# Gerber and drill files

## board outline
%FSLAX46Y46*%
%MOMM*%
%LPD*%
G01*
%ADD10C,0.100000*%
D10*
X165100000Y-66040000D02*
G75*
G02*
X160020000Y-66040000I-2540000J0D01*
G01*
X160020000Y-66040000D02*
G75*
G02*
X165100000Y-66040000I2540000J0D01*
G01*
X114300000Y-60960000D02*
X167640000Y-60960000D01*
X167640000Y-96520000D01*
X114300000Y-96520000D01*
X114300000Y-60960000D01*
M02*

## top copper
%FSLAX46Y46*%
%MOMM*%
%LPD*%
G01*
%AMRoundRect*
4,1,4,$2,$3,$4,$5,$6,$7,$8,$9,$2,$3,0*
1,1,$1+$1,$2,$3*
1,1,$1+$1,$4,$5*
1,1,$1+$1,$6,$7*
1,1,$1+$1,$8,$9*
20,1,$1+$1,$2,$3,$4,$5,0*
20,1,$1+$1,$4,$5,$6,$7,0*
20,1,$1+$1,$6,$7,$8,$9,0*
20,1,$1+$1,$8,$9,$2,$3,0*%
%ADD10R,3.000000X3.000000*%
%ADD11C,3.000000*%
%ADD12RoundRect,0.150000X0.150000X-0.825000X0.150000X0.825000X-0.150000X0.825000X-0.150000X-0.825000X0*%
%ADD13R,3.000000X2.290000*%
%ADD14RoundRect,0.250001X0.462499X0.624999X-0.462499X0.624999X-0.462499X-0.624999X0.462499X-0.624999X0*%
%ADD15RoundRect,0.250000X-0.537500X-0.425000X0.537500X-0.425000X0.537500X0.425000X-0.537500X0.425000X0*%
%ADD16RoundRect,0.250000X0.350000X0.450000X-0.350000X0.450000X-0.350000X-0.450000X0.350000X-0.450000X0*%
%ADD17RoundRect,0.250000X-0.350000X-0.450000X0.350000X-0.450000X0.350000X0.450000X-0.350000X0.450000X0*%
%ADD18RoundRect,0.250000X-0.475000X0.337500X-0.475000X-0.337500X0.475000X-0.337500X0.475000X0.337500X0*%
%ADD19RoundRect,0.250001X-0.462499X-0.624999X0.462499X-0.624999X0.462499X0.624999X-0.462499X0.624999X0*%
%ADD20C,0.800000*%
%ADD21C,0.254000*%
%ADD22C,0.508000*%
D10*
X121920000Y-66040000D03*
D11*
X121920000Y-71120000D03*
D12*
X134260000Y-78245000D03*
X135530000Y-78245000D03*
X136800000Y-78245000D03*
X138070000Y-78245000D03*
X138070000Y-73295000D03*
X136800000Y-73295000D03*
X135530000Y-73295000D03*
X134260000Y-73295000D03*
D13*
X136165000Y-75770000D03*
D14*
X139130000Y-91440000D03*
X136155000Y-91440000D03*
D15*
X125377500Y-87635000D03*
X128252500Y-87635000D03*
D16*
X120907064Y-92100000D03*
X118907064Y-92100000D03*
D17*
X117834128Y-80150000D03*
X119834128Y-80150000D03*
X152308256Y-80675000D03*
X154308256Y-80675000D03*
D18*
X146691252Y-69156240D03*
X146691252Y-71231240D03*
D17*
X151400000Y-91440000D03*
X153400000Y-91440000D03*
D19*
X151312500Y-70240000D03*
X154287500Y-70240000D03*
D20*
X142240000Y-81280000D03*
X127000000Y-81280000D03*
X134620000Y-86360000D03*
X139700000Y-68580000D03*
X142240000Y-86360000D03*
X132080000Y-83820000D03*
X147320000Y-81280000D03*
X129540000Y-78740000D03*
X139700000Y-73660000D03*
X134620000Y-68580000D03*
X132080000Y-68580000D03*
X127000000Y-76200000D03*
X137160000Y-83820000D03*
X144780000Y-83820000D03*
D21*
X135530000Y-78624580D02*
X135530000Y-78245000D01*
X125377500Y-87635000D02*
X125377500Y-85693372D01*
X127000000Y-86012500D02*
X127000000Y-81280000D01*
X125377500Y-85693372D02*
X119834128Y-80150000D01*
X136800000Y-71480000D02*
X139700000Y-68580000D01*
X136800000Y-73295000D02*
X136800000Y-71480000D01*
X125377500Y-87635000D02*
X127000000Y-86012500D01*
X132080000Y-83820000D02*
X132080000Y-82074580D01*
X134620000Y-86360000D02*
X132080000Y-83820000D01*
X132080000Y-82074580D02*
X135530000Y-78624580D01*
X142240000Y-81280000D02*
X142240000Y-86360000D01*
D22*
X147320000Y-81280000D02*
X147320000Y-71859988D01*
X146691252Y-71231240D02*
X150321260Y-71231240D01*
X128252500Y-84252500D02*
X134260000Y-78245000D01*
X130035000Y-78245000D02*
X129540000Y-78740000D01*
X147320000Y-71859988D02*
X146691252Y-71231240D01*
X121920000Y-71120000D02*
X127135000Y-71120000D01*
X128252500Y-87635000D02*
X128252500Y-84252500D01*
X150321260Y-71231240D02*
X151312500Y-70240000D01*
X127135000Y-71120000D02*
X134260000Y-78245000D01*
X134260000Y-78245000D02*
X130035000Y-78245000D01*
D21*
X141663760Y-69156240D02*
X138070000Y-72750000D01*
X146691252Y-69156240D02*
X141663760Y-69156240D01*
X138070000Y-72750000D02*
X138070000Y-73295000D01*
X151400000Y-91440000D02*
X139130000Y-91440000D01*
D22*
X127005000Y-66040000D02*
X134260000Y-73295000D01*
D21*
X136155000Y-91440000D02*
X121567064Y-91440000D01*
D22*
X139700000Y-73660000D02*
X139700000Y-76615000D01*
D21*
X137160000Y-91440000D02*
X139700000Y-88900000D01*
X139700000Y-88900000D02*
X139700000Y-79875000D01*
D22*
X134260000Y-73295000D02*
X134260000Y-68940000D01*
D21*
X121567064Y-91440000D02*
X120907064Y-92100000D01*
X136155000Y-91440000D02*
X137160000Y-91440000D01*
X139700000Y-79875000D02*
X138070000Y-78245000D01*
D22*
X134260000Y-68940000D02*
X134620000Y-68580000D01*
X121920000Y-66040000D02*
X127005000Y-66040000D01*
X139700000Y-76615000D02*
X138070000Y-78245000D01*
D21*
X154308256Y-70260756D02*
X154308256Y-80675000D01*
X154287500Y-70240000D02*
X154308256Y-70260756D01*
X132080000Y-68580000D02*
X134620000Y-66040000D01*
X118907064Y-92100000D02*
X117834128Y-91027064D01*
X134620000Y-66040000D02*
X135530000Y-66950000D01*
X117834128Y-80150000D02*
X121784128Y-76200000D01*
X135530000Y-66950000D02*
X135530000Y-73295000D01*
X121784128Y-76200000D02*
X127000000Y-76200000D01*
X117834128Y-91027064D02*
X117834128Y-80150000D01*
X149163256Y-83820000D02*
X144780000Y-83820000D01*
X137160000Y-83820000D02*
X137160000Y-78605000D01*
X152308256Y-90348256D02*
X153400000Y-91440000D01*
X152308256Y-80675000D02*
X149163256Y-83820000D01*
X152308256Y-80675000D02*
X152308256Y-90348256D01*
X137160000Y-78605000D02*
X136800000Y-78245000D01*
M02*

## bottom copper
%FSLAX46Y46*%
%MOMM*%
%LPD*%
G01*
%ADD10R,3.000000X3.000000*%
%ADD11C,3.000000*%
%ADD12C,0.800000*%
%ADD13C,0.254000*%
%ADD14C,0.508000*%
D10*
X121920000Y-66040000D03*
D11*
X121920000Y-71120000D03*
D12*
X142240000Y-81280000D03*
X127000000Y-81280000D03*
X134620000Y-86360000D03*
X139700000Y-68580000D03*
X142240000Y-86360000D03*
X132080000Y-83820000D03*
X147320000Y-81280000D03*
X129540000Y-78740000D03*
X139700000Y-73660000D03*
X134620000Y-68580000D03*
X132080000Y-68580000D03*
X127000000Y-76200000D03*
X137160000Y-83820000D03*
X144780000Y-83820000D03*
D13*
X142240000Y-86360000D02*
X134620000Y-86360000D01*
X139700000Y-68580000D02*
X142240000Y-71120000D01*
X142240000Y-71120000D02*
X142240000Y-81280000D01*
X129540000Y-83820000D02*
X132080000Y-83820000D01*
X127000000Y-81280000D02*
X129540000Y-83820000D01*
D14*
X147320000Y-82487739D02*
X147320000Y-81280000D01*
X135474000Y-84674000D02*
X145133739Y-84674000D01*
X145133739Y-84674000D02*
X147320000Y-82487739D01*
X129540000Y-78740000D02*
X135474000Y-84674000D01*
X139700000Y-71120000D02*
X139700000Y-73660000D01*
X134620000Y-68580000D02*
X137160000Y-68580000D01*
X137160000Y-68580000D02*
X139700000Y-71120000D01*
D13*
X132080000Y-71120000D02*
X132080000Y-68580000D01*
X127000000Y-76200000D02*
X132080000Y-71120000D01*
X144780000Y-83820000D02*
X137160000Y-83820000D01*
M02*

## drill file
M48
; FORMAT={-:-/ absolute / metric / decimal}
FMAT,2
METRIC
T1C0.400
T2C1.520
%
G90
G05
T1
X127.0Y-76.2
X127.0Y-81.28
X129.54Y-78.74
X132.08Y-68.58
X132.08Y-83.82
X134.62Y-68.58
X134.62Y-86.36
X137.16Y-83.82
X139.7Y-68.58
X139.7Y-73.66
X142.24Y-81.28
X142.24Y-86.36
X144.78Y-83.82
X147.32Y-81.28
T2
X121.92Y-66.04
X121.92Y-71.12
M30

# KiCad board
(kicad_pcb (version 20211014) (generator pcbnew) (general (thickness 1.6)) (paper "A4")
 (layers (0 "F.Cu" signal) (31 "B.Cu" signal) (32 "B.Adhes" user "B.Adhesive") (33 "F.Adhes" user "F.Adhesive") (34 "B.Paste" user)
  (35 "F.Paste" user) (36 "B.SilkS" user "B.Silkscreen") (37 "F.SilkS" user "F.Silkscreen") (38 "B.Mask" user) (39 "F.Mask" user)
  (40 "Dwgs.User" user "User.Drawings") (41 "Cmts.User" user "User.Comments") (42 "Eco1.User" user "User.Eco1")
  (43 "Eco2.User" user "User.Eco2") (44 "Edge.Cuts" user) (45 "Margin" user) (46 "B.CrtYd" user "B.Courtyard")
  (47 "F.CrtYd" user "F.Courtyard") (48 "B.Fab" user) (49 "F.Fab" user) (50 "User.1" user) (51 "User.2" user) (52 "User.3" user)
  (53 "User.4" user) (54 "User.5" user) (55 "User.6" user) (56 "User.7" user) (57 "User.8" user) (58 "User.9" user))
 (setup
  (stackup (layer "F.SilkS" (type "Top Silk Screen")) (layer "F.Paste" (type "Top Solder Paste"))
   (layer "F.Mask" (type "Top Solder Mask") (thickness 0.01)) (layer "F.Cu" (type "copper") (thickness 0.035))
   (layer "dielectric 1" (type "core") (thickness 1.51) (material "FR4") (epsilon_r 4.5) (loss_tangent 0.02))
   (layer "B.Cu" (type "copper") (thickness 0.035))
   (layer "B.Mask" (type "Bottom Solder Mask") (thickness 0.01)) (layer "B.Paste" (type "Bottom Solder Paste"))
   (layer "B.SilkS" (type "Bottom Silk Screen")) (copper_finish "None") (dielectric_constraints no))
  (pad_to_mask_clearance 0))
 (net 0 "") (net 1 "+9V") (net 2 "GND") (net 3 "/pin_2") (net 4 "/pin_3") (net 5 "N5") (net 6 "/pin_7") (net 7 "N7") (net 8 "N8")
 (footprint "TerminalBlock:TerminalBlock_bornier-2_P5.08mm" (layer "F.Cu") (at 121.92 66.04 -90)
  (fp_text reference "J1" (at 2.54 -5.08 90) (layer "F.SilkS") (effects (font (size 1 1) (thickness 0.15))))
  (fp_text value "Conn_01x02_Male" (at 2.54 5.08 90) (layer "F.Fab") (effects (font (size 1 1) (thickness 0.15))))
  (pad "1" thru_hole rect (at 0 0 270) (size 3 3) (drill 1.52) (layers *.Cu *.Mask) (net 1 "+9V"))
  (pad "2" thru_hole circle (at 5.08 0 270) (size 3 3) (drill 1.52) (layers *.Cu *.Mask) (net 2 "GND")))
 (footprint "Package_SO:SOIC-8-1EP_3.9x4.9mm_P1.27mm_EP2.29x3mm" (layer "F.Cu") (at 136.165 75.77 90)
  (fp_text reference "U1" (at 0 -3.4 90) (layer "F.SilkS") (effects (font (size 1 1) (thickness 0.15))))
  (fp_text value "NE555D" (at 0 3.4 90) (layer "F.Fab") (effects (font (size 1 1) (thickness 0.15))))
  (pad "" smd roundrect (at -0.57 -0.75 90) (size 0.92 1.21) (layers "F.Paste") (roundrect_rratio 0.25))
  (pad "" smd roundrect (at 0.57 -0.75 90) (size 0.92 1.21) (layers "F.Paste") (roundrect_rratio 0.25))
  (pad "" smd roundrect (at 0.57 0.75 90) (size 0.92 1.21) (layers "F.Paste") (roundrect_rratio 0.25))
  (pad "" smd roundrect (at -0.57 0.75 90) (size 0.92 1.21) (layers "F.Paste") (roundrect_rratio 0.25))
  (pad "1" smd roundrect (at -2.475 -1.905 90) (size 1.95 0.6) (layers "F.Cu" "F.Paste" "F.Mask") (roundrect_rratio 0.25) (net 2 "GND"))
  (pad "2" smd roundrect (at -2.475 -0.635 90) (size 1.95 0.6) (layers "F.Cu" "F.Paste" "F.Mask") (roundrect_rratio 0.25) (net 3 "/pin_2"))
  (pad "3" smd roundrect (at -2.475 0.635 90) (size 1.95 0.6) (layers "F.Cu" "F.Paste" "F.Mask") (roundrect_rratio 0.25) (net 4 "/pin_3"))
  (pad "4" smd roundrect (at -2.475 1.905 90) (size 1.95 0.6) (layers "F.Cu" "F.Paste" "F.Mask") (roundrect_rratio 0.25) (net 1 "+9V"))
  (pad "5" smd roundrect (at 2.475 1.905 90) (size 1.95 0.6) (layers "F.Cu" "F.Paste" "F.Mask") (roundrect_rratio 0.25) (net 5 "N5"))
  (pad "6" smd roundrect (at 2.475 0.635 90) (size 1.95 0.6) (layers "F.Cu" "F.Paste" "F.Mask") (roundrect_rratio 0.25) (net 3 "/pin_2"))
  (pad "7" smd roundrect (at 2.475 -0.635 90) (size 1.95 0.6) (layers "F.Cu" "F.Paste" "F.Mask") (roundrect_rratio 0.25) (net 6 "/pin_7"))
  (pad "8" smd roundrect (at 2.475 -1.905 90) (size 1.95 0.6) (layers "F.Cu" "F.Paste" "F.Mask") (roundrect_rratio 0.25) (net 1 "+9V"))
  (pad "9" smd rect (at 0 0 90) (size 2.29 3) (layers "F.Cu" "F.Mask")))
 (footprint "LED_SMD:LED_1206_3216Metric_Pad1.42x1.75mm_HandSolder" (layer "F.Cu") (at 137.6425 91.44 180)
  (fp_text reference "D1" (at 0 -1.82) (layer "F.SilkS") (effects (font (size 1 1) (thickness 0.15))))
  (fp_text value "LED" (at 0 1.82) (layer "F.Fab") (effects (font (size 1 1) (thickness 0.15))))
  (pad "1" smd roundrect (at -1.4875 0 180) (size 1.425 1.75) (layers "F.Cu" "F.Paste" "F.Mask") (roundrect_rratio 0.175439) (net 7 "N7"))
  (pad "2" smd roundrect (at 1.4875 0 180) (size 1.425 1.75) (layers "F.Cu" "F.Paste" "F.Mask") (roundrect_rratio 0.175439) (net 1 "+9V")))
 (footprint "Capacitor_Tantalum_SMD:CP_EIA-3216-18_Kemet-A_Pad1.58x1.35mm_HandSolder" (layer "F.Cu") (at 126.815 87.635)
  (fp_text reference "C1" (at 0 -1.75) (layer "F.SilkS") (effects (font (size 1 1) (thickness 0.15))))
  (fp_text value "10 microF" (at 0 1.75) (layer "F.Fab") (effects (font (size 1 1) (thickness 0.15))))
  (pad "1" smd roundrect (at -1.4375 0) (size 1.575 1.35) (layers "F.Cu" "F.Paste" "F.Mask") (roundrect_rratio 0.185185) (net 3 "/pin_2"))
  (pad "2" smd roundrect (at 1.4375 0) (size 1.575 1.35) (layers "F.Cu" "F.Paste" "F.Mask") (roundrect_rratio 0.185185) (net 2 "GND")))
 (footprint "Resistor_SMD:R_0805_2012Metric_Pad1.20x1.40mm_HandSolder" (layer "F.Cu") (at 119.907064 92.1 180)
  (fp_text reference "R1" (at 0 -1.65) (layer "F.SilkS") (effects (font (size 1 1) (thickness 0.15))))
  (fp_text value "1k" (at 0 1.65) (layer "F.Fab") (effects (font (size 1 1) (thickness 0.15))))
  (pad "1" smd roundrect (at -1 0 180) (size 1.2 1.4) (layers "F.Cu" "F.Paste" "F.Mask") (roundrect_rratio 0.208333) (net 1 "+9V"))
  (pad "2" smd roundrect (at 1 0 180) (size 1.2 1.4) (layers "F.Cu" "F.Paste" "F.Mask") (roundrect_rratio 0.208333) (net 6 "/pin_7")))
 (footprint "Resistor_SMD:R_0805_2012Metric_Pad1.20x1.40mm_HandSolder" (layer "F.Cu") (at 118.834128 80.15)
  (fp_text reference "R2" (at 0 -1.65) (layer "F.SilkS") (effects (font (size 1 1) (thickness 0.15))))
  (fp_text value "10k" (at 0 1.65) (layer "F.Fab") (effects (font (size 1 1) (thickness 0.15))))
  (pad "1" smd roundrect (at -1 0) (size 1.2 1.4) (layers "F.Cu" "F.Paste" "F.Mask") (roundrect_rratio 0.208333) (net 6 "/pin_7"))
  (pad "2" smd roundrect (at 1 0) (size 1.2 1.4) (layers "F.Cu" "F.Paste" "F.Mask") (roundrect_rratio 0.208333) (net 3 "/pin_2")))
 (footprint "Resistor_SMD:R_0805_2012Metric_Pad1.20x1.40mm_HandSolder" (layer "F.Cu") (at 153.308256 80.675)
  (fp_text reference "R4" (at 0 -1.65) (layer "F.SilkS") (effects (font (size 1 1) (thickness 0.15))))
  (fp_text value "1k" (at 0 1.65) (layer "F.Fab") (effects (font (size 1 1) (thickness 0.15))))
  (pad "1" smd roundrect (at -1 0) (size 1.2 1.4) (layers "F.Cu" "F.Paste" "F.Mask") (roundrect_rratio 0.208333) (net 4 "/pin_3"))
  (pad "2" smd roundrect (at 1 0) (size 1.2 1.4) (layers "F.Cu" "F.Paste" "F.Mask") (roundrect_rratio 0.208333) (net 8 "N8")))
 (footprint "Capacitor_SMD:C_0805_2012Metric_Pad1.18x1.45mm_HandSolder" (layer "F.Cu") (at 146.691252 70.19374 -90)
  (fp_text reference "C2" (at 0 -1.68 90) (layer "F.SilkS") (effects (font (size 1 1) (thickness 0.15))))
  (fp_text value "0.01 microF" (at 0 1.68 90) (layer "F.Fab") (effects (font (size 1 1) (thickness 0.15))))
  (pad "1" smd roundrect (at -1.0375 0 270) (size 1.175 1.45) (layers "F.Cu" "F.Paste" "F.Mask") (roundrect_rratio 0.212766) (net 5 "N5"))
  (pad "2" smd roundrect (at 1.0375 0 270) (size 1.175 1.45) (layers "F.Cu" "F.Paste" "F.Mask") (roundrect_rratio 0.212766) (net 2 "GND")))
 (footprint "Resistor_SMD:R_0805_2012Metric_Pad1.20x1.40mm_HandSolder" (layer "F.Cu") (at 152.4 91.44)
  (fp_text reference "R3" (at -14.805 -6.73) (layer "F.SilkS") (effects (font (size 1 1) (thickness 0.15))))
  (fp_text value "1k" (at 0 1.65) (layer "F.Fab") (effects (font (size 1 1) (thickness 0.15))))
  (pad "1" smd roundrect (at -1 0) (size 1.2 1.4) (layers "F.Cu" "F.Paste" "F.Mask") (roundrect_rratio 0.208333) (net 7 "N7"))
  (pad "2" smd roundrect (at 1 0) (size 1.2 1.4) (layers "F.Cu" "F.Paste" "F.Mask") (roundrect_rratio 0.208333) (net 4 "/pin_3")))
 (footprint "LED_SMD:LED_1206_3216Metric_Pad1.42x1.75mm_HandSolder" (layer "F.Cu") (at 152.8 70.24)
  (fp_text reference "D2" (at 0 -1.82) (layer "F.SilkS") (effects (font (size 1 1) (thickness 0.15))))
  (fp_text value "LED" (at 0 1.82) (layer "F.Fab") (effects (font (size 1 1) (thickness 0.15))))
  (pad "1" smd roundrect (at -1.4875 0) (size 1.425 1.75) (layers "F.Cu" "F.Paste" "F.Mask") (roundrect_rratio 0.175439) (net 2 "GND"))
  (pad "2" smd roundrect (at 1.4875 0) (size 1.425 1.75) (layers "F.Cu" "F.Paste" "F.Mask") (roundrect_rratio 0.175439) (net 8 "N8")))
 (gr_circle (center 162.56 66.04) (end 162.56 68.58) (layer "Edge.Cuts") (width 0.1) (fill none))
 (gr_rect (start 114.3 60.96) (end 167.64 96.52) (layer "Edge.Cuts") (width 0.1) (fill none))
 (segment (start 135.53 78.62458) (end 135.53 78.245) (width 0.254) (layer "F.Cu") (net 3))
 (segment (start 125.3775 87.635) (end 125.3775 85.693372) (width 0.254) (layer "F.Cu") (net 3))
 (segment (start 127 86.0125) (end 127 81.28) (width 0.254) (layer "F.Cu") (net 3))
 (segment (start 125.3775 85.693372) (end 119.834128 80.15) (width 0.254) (layer "F.Cu") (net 3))
 (segment (start 136.8 71.48) (end 139.7 68.58) (width 0.254) (layer "F.Cu") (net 3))
 (segment (start 136.8 73.295) (end 136.8 71.48) (width 0.254) (layer "F.Cu") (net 3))
 (segment (start 125.3775 87.635) (end 127 86.0125) (width 0.254) (layer "F.Cu") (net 3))
 (segment (start 132.08 83.82) (end 132.08 82.07458) (width 0.254) (layer "F.Cu") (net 3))
 (segment (start 134.62 86.36) (end 132.08 83.82) (width 0.254) (layer "F.Cu") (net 3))
 (segment (start 132.08 82.07458) (end 135.53 78.62458) (width 0.254) (layer "F.Cu") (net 3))
 (segment (start 142.24 81.28) (end 142.24 86.36) (width 0.254) (layer "F.Cu") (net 3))
 (via (at 142.24 81.28) (size 0.8) (drill 0.4) (layers "F.Cu" "B.Cu") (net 3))
 (via (at 127 81.28) (size 0.8) (drill 0.4) (layers "F.Cu" "B.Cu") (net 3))
 (via (at 134.62 86.36) (size 0.8) (drill 0.4) (layers "F.Cu" "B.Cu") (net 3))
 (via (at 139.7 68.58) (size 0.8) (drill 0.4) (layers "F.Cu" "B.Cu") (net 3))
 (via (at 142.24 86.36) (size 0.8) (drill 0.4) (layers "F.Cu" "B.Cu") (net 3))
 (via (at 132.08 83.82) (size 0.8) (drill 0.4) (layers "F.Cu" "B.Cu") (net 3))
 (segment (start 142.24 86.36) (end 134.62 86.36) (width 0.254) (layer "B.Cu") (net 3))
 (segment (start 139.7 68.58) (end 142.24 71.12) (width 0.254) (layer "B.Cu") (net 3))
 (segment (start 142.24 71.12) (end 142.24 81.28) (width 0.254) (layer "B.Cu") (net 3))
 (segment (start 129.54 83.82) (end 132.08 83.82) (width 0.254) (layer "B.Cu") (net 3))
 (segment (start 127 81.28) (end 129.54 83.82) (width 0.254) (layer "B.Cu") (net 3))
 (segment (start 147.32 81.28) (end 147.32 71.859988) (width 0.508) (layer "F.Cu") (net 2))
 (segment (start 146.691252 71.23124) (end 150.32126 71.23124) (width 0.508) (layer "F.Cu") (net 2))
 (segment (start 128.2525 84.2525) (end 134.26 78.245) (width 0.508) (layer "F.Cu") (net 2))
 (segment (start 130.035 78.245) (end 129.54 78.74) (width 0.508) (layer "F.Cu") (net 2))
 (segment (start 147.32 71.859988) (end 146.691252 71.23124) (width 0.508) (layer "F.Cu") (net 2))
 (segment (start 121.92 71.12) (end 127.135 71.12) (width 0.508) (layer "F.Cu") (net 2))
 (segment (start 128.2525 87.635) (end 128.2525 84.2525) (width 0.508) (layer "F.Cu") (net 2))
 (segment (start 150.32126 71.23124) (end 151.3125 70.24) (width 0.508) (layer "F.Cu") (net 2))
 (segment (start 127.135 71.12) (end 134.26 78.245) (width 0.508) (layer "F.Cu") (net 2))
 (segment (start 134.26 78.245) (end 130.035 78.245) (width 0.508) (layer "F.Cu") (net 2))
 (via (at 147.32 81.28) (size 0.8) (drill 0.4) (layers "F.Cu" "B.Cu") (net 2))
 (via (at 129.54 78.74) (size 0.8) (drill 0.4) (layers "F.Cu" "B.Cu") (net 2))
 (segment (start 147.32 82.487739) (end 147.32 81.28) (width 0.508) (layer "B.Cu") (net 2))
 (segment (start 135.474 84.674) (end 145.133739 84.674) (width 0.508) (layer "B.Cu") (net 2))
 (segment (start 145.133739 84.674) (end 147.32 82.487739) (width 0.508) (layer "B.Cu") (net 2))
 (segment (start 129.54 78.74) (end 135.474 84.674) (width 0.508) (layer "B.Cu") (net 2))
 (segment (start 141.66376 69.15624) (end 138.07 72.75) (width 0.254) (layer "F.Cu") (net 5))
 (segment (start 146.691252 69.15624) (end 141.66376 69.15624) (width 0.254) (layer "F.Cu") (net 5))
 (segment (start 138.07 72.75) (end 138.07 73.295) (width 0.254) (layer "F.Cu") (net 5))
 (segment (start 151.4 91.44) (end 139.13 91.44) (width 0.254) (layer "F.Cu") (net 7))
 (segment (start 127.005 66.04) (end 134.26 73.295) (width 0.508) (layer "F.Cu") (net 1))
 (segment (start 136.155 91.44) (end 121.567064 91.44) (width 0.254) (layer "F.Cu") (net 1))
 (segment (start 139.7 73.66) (end 139.7 76.615) (width 0.508) (layer "F.Cu") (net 1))
 (segment (start 137.16 91.44) (end 139.7 88.9) (width 0.254) (layer "F.Cu") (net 1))
 (segment (start 139.7 88.9) (end 139.7 79.875) (width 0.254) (layer "F.Cu") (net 1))
 (segment (start 134.26 73.295) (end 134.26 68.94) (width 0.508) (layer "F.Cu") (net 1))
 (segment (start 121.567064 91.44) (end 120.907064 92.1) (width 0.254) (layer "F.Cu") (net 1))
 (segment (start 136.155 91.44) (end 137.16 91.44) (width 0.254) (layer "F.Cu") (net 1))
 (segment (start 139.7 79.875) (end 138.07 78.245) (width 0.254) (layer "F.Cu") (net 1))
 (segment (start 134.26 68.94) (end 134.62 68.58) (width 0.508) (layer "F.Cu") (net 1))
 (segment (start 121.92 66.04) (end 127.005 66.04) (width 0.508) (layer "F.Cu") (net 1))
 (segment (start 139.7 76.615) (end 138.07 78.245) (width 0.508) (layer "F.Cu") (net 1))
 (via (at 139.7 73.66) (size 0.8) (drill 0.4) (layers "F.Cu" "B.Cu") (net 1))
 (via (at 134.62 68.58) (size 0.8) (drill 0.4) (layers "F.Cu" "B.Cu") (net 1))
 (segment (start 139.7 71.12) (end 139.7 73.66) (width 0.508) (layer "B.Cu") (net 1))
 (segment (start 134.62 68.58) (end 137.16 68.58) (width 0.508) (layer "B.Cu") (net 1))
 (segment (start 137.16 68.58) (end 139.7 71.12) (width 0.508) (layer "B.Cu") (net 1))
 (segment (start 154.308256 70.260756) (end 154.308256 80.675) (width 0.254) (layer "F.Cu") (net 8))
 (segment (start 154.2875 70.24) (end 154.308256 70.260756) (width 0.254) (layer "F.Cu") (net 8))
 (segment (start 132.08 68.58) (end 134.62 66.04) (width 0.254) (layer "F.Cu") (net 6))
 (segment (start 118.907064 92.1) (end 117.834128 91.027064) (width 0.254) (layer "F.Cu") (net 6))
 (segment (start 134.62 66.04) (end 135.53 66.95) (width 0.254) (layer "F.Cu") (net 6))
 (segment (start 117.834128 80.15) (end 121.784128 76.2) (width 0.254) (layer "F.Cu") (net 6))
 (segment (start 135.53 66.95) (end 135.53 73.295) (width 0.254) (layer "F.Cu") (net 6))
 (segment (start 121.784128 76.2) (end 127 76.2) (width 0.254) (layer "F.Cu") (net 6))
 (segment (start 117.834128 91.027064) (end 117.834128 80.15) (width 0.254) (layer "F.Cu") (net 6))
 (via (at 132.08 68.58) (size 0.8) (drill 0.4) (layers "F.Cu" "B.Cu") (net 6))
 (via (at 127 76.2) (size 0.8) (drill 0.4) (layers "F.Cu" "B.Cu") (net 6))
 (segment (start 132.08 71.12) (end 132.08 68.58) (width 0.254) (layer "B.Cu") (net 6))
 (segment (start 127 76.2) (end 132.08 71.12) (width 0.254) (layer "B.Cu") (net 6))
 (segment (start 149.163256 83.82) (end 144.78 83.82) (width 0.254) (layer "F.Cu") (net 4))
 (segment (start 137.16 83.82) (end 137.16 78.605) (width 0.254) (layer "F.Cu") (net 4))
 (segment (start 152.308256 90.348256) (end 153.4 91.44) (width 0.254) (layer "F.Cu") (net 4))
 (segment (start 152.308256 80.675) (end 149.163256 83.82) (width 0.254) (layer "F.Cu") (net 4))
 (segment (start 152.308256 80.675) (end 152.308256 90.348256) (width 0.254) (layer "F.Cu") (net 4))
 (segment (start 137.16 78.605) (end 136.8 78.245) (width 0.254) (layer "F.Cu") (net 4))
 (via (at 137.16 83.82) (size 0.8) (drill 0.4) (layers "F.Cu" "B.Cu") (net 4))
 (via (at 144.78 83.82) (size 0.8) (drill 0.4) (layers "F.Cu" "B.Cu") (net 4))
 (segment (start 144.78 83.82) (end 137.16 83.82) (width 0.254) (layer "B.Cu") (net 4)))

